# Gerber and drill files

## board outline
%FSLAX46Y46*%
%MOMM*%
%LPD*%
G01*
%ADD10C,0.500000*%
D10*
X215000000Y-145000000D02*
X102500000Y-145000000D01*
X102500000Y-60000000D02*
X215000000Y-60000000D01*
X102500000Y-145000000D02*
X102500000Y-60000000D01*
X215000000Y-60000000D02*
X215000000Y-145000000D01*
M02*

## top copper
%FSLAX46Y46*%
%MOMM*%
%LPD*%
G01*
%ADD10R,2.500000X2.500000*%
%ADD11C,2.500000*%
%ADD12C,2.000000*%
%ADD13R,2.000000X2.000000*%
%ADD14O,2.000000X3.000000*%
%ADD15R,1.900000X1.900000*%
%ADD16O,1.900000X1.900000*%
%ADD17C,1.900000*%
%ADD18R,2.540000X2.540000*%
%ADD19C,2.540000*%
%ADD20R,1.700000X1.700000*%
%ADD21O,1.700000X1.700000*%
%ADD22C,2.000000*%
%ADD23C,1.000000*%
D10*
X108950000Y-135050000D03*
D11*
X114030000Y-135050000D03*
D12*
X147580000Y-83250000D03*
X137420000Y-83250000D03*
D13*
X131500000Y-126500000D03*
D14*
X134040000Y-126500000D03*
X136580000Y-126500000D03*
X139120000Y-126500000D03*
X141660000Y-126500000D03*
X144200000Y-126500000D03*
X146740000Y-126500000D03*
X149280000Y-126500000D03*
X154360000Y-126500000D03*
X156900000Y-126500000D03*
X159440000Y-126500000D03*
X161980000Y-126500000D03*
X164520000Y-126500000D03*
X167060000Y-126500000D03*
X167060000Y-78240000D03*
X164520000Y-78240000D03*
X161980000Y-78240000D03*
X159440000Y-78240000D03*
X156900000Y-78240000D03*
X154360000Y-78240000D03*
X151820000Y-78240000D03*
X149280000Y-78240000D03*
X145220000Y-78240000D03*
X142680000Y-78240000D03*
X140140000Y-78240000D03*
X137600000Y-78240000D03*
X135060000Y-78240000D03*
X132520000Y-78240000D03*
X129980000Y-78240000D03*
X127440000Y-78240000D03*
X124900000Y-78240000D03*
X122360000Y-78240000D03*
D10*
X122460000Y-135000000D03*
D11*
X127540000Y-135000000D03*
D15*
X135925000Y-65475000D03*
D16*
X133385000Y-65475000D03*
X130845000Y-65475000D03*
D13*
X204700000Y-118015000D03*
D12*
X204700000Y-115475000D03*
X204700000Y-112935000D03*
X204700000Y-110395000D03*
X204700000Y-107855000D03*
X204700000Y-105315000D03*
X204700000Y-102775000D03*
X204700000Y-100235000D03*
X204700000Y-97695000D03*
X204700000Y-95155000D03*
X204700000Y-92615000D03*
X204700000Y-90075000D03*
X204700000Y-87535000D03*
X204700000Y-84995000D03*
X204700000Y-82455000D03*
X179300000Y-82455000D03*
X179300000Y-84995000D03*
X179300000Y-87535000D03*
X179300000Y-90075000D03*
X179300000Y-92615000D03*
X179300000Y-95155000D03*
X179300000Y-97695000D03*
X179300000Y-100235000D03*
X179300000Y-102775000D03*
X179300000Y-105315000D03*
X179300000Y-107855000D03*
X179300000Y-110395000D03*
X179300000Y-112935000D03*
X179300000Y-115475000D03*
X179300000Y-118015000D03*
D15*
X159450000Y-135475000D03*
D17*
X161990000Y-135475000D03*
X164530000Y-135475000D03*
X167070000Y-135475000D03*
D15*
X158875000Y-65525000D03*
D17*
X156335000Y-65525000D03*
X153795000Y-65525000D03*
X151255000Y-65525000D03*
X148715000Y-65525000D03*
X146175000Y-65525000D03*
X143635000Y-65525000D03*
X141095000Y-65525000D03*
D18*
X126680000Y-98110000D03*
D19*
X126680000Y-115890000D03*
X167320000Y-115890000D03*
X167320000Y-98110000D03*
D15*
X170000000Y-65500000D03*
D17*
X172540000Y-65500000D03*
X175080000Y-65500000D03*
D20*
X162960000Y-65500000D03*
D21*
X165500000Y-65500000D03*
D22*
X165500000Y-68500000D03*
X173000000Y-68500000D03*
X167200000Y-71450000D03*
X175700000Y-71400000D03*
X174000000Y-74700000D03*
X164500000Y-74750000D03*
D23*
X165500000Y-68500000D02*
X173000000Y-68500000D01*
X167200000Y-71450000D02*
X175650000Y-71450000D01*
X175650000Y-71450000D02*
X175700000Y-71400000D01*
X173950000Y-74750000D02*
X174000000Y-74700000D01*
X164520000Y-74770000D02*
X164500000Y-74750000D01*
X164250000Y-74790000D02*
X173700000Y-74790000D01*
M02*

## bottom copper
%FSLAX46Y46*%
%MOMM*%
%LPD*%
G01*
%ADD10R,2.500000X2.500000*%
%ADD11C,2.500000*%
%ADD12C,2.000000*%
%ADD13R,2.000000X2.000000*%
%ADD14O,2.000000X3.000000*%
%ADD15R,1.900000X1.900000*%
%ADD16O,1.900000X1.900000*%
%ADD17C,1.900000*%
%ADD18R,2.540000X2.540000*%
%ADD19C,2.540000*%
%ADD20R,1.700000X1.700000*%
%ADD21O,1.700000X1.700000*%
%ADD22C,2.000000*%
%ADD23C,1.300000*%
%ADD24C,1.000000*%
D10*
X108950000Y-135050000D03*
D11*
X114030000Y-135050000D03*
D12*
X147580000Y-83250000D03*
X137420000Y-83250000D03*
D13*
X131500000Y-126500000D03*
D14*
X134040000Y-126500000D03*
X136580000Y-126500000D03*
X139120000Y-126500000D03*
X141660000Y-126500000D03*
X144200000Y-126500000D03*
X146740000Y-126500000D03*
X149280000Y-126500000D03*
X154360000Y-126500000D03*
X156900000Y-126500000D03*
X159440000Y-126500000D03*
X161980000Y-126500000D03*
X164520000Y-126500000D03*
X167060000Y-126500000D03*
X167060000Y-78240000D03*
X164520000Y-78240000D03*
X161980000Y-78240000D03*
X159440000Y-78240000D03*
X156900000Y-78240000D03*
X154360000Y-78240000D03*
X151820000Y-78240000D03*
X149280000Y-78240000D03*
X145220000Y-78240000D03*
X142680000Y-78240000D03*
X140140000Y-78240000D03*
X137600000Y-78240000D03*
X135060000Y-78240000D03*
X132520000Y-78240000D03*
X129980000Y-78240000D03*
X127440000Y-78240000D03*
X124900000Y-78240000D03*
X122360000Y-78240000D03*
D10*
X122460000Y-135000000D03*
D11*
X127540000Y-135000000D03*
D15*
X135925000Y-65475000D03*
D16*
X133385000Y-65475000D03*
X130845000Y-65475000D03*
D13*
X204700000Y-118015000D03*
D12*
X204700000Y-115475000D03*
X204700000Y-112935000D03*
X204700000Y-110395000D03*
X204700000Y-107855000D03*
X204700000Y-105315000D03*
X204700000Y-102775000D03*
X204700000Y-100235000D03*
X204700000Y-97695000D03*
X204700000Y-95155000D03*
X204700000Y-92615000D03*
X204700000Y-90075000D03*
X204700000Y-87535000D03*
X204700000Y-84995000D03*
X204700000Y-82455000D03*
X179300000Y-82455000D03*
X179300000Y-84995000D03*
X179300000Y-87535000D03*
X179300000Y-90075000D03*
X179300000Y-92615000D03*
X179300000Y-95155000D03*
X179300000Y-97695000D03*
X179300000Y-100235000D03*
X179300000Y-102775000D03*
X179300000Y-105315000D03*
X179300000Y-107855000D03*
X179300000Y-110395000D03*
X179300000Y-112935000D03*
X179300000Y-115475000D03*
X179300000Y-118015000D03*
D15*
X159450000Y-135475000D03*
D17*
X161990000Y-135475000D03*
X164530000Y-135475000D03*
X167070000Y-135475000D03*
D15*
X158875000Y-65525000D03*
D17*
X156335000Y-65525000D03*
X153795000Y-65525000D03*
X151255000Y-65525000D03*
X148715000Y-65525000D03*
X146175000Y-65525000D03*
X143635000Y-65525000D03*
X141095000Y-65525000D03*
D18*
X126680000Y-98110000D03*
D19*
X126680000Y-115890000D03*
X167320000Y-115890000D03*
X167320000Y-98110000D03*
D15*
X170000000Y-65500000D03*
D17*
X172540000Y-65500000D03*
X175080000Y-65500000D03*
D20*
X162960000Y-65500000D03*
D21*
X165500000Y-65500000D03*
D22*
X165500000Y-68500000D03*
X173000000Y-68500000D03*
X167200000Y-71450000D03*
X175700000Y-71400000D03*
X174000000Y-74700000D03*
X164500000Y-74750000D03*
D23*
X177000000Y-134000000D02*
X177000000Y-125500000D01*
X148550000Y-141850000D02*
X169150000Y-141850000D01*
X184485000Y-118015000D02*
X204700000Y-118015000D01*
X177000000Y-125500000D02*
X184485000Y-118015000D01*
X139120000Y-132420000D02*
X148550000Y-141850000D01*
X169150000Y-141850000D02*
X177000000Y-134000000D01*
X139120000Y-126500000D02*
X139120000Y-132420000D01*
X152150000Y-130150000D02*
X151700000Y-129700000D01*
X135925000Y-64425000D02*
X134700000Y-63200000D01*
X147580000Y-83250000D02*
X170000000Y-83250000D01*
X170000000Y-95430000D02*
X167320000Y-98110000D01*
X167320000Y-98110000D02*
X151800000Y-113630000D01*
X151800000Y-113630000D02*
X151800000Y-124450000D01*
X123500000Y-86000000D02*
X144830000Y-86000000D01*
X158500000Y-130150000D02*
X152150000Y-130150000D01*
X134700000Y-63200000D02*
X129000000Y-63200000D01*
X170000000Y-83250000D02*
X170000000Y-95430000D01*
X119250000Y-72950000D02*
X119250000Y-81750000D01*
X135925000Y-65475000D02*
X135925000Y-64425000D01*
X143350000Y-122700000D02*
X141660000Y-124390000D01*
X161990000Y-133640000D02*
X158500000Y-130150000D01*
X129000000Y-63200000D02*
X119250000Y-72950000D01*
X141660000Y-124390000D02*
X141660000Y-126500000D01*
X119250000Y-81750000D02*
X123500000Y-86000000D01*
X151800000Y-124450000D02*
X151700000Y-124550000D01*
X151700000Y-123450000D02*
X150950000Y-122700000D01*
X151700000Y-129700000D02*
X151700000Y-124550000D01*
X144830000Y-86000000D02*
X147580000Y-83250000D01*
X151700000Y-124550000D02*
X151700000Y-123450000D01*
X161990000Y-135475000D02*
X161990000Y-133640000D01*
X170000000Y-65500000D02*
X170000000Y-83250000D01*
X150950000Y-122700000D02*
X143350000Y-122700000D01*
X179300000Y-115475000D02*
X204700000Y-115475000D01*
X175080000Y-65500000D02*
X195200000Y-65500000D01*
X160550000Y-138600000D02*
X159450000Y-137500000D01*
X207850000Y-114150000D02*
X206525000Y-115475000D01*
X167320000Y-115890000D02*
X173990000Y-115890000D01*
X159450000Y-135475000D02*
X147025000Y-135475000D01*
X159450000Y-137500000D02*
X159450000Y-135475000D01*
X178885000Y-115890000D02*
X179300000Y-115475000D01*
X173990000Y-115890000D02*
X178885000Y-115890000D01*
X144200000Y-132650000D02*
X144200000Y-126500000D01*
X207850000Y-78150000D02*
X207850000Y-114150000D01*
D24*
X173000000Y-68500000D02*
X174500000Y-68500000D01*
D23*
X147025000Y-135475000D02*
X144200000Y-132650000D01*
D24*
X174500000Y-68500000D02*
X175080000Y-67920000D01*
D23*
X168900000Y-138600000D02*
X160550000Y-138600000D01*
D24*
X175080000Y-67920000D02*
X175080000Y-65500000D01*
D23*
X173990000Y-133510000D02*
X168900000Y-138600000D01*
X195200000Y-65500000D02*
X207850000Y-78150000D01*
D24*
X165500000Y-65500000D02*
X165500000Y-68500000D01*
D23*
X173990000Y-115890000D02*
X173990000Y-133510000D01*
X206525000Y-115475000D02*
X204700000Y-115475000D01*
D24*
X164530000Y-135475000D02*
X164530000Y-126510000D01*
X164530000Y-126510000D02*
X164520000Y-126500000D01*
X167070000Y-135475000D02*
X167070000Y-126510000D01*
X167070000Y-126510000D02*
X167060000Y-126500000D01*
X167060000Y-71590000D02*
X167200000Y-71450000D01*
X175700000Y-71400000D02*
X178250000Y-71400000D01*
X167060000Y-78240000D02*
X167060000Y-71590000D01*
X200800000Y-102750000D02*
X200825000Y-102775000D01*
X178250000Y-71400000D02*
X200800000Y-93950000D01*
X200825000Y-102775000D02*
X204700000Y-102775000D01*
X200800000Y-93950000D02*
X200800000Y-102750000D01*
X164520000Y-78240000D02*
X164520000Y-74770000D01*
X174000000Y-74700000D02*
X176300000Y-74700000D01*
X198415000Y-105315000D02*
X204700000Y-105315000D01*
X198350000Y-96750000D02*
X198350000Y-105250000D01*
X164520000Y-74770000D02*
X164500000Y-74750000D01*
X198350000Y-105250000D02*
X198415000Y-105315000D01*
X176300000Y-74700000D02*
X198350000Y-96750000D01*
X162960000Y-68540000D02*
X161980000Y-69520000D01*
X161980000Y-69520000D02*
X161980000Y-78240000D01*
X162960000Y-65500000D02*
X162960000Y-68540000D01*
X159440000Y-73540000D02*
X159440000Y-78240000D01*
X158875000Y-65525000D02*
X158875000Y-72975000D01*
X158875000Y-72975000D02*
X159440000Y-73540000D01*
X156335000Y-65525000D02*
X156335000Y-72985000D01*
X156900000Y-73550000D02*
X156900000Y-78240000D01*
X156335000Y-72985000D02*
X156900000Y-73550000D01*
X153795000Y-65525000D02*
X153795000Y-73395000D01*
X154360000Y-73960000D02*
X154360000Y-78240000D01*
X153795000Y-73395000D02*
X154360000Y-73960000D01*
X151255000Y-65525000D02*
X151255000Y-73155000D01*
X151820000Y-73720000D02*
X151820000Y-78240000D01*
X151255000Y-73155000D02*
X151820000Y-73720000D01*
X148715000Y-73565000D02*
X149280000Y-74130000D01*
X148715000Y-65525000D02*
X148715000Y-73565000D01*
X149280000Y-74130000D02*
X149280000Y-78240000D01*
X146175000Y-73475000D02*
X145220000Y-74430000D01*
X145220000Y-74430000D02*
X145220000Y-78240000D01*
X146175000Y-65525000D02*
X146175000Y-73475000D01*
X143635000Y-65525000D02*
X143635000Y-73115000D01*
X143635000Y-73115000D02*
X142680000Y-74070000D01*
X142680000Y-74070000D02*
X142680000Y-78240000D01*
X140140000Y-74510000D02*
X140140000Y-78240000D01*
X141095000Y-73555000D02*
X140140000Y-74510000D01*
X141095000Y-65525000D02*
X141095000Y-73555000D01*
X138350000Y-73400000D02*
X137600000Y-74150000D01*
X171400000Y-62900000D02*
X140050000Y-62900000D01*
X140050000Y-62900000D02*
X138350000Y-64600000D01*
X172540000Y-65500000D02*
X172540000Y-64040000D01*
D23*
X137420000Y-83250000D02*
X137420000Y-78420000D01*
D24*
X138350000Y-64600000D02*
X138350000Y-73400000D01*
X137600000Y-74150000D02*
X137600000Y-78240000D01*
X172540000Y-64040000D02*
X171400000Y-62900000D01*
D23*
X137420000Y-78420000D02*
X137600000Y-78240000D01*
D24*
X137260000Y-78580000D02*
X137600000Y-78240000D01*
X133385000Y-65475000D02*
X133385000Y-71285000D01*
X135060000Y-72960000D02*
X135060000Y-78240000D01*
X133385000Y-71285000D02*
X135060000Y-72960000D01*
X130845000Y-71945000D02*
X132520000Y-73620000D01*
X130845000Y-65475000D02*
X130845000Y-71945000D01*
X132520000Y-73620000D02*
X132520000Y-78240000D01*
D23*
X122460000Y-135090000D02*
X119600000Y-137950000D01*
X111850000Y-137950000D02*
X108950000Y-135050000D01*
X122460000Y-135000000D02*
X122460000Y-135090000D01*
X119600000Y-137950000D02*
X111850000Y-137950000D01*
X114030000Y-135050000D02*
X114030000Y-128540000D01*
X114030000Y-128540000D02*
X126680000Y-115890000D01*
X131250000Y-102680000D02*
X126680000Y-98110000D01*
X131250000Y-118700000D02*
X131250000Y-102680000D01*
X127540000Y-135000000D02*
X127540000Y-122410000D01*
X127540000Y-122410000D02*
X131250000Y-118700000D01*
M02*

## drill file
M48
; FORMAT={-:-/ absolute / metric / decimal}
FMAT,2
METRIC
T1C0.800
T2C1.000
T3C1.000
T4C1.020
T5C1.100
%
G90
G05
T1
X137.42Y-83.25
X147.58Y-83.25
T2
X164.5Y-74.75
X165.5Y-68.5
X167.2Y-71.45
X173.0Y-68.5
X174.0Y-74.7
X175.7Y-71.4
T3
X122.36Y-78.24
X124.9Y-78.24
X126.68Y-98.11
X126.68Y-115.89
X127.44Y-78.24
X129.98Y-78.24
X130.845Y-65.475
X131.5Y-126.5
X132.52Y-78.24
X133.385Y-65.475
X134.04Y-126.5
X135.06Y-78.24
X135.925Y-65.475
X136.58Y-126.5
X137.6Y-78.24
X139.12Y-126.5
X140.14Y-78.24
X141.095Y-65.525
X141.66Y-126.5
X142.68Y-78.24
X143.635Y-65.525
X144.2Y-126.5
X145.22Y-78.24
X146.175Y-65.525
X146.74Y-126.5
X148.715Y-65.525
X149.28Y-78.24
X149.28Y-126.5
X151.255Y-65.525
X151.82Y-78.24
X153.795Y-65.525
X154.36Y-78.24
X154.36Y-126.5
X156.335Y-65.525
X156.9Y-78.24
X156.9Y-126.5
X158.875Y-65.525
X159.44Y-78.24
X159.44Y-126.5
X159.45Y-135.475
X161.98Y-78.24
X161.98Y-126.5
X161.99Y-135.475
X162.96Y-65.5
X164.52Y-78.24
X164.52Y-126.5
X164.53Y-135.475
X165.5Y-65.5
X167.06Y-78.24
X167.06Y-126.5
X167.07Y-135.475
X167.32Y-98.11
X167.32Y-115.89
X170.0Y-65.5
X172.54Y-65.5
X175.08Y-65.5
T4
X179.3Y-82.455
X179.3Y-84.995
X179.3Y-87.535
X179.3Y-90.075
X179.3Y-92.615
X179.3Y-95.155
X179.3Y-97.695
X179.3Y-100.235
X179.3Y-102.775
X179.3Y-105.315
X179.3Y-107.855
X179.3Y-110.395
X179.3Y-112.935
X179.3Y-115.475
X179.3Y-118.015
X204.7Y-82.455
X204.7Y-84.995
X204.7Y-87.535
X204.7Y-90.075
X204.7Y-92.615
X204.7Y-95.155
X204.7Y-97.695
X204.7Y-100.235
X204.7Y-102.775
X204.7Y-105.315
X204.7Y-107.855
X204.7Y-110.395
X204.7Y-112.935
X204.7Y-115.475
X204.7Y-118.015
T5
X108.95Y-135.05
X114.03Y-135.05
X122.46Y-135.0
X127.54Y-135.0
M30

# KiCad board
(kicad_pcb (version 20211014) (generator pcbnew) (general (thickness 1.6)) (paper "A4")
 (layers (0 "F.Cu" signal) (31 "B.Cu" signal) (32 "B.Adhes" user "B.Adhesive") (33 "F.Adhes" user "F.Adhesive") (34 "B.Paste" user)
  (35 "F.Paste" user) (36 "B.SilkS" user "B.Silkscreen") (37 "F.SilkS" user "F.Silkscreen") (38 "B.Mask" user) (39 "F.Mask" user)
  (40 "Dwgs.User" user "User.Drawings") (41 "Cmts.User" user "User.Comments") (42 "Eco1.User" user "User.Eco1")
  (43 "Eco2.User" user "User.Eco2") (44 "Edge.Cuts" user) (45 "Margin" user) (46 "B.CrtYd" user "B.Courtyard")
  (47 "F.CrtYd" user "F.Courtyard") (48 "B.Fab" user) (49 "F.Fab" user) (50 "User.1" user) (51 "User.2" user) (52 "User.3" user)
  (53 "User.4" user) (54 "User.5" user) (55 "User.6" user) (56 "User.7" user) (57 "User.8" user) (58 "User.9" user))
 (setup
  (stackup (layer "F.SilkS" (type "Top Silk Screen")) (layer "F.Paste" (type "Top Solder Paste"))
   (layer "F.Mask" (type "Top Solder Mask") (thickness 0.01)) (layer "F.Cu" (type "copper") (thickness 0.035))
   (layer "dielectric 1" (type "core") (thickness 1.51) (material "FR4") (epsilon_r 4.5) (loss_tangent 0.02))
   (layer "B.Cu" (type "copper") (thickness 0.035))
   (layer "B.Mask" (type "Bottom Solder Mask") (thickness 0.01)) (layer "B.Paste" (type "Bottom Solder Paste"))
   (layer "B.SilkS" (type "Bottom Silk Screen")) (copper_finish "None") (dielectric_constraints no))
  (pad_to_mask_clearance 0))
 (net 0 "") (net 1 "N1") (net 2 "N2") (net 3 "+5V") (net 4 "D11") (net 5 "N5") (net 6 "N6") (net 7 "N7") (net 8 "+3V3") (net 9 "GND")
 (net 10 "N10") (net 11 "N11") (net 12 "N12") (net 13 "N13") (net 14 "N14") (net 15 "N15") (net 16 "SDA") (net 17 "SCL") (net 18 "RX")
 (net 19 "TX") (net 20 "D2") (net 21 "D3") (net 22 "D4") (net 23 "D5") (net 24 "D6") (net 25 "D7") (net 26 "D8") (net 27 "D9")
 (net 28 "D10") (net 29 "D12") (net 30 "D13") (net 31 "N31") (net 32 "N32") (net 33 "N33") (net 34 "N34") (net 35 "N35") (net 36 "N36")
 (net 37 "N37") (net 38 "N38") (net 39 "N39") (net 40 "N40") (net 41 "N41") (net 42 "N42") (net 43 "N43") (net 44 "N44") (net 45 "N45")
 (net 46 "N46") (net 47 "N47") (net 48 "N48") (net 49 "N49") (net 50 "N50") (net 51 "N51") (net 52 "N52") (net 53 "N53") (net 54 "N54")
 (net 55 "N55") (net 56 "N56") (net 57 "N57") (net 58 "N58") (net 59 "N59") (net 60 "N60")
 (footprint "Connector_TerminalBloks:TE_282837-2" (layer "F.Cu") (at 111.49 135.05)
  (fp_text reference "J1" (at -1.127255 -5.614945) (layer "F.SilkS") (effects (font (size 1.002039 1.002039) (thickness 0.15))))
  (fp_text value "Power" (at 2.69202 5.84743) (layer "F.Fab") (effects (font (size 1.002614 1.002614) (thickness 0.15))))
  (pad "1" thru_hole rect (at -2.54 0) (size 2.5 2.5) (drill 1.1) (layers *.Cu *.Mask) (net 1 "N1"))
  (pad "2" thru_hole circle (at 2.54 0) (size 2.5 2.5) (drill 1.1) (layers *.Cu *.Mask) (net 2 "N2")))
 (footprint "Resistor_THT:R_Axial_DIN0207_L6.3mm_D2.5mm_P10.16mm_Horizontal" (layer "F.Cu") (at 147.58 83.25 180)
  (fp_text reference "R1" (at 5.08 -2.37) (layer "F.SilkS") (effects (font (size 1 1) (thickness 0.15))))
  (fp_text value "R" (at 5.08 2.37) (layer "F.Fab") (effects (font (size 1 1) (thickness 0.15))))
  (pad "1" thru_hole circle (at 0 0 180) (size 2 2) (drill 0.8) (layers *.Cu *.Mask) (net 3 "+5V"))
  (pad "2" thru_hole circle (at 10.16 0 180) (size 2 2) (drill 0.8) (layers *.Cu *.Mask) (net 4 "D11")))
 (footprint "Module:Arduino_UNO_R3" (layer "F.Cu") (at 131.5 80.5)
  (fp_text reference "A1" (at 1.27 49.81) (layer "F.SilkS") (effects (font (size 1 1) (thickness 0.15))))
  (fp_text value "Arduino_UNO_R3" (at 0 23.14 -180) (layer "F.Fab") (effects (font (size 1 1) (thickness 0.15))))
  (pad "1" thru_hole rect (at 0 46 90) (size 2 2) (drill 1) (layers *.Cu *.Mask) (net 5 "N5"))
  (pad "2" thru_hole oval (at 2.54 46 90) (size 3 2) (drill 1) (layers *.Cu *.Mask) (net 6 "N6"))
  (pad "3" thru_hole oval (at 5.08 46 90) (size 3 2) (drill 1) (layers *.Cu *.Mask) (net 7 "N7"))
  (pad "4" thru_hole oval (at 7.62 46 90) (size 3 2) (drill 1) (layers *.Cu *.Mask) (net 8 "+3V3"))
  (pad "5" thru_hole oval (at 10.16 46 90) (size 3 2) (drill 1) (layers *.Cu *.Mask) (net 3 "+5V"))
  (pad "6" thru_hole oval (at 12.7 46 90) (size 3 2) (drill 1) (layers *.Cu *.Mask) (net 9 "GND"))
  (pad "7" thru_hole oval (at 15.24 46 90) (size 3 2) (drill 1) (layers *.Cu *.Mask) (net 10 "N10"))
  (pad "8" thru_hole oval (at 17.78 46 90) (size 3 2) (drill 1) (layers *.Cu *.Mask) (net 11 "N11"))
  (pad "9" thru_hole oval (at 22.86 46 90) (size 3 2) (drill 1) (layers *.Cu *.Mask) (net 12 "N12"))
  (pad "10" thru_hole oval (at 25.4 46 90) (size 3 2) (drill 1) (layers *.Cu *.Mask) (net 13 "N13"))
  (pad "11" thru_hole oval (at 27.94 46 90) (size 3 2) (drill 1) (layers *.Cu *.Mask) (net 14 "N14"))
  (pad "12" thru_hole oval (at 30.48 46 90) (size 3 2) (drill 1) (layers *.Cu *.Mask) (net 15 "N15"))
  (pad "13" thru_hole oval (at 33.02 46 90) (size 3 2) (drill 1) (layers *.Cu *.Mask) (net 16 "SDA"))
  (pad "14" thru_hole oval (at 35.56 46 90) (size 3 2) (drill 1) (layers *.Cu *.Mask) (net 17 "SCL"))
  (pad "15" thru_hole oval (at 35.56 -2.26 90) (size 3 2) (drill 1) (layers *.Cu *.Mask) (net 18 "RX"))
  (pad "16" thru_hole oval (at 33.02 -2.26 90) (size 3 2) (drill 1) (layers *.Cu *.Mask) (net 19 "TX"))
  (pad "17" thru_hole oval (at 30.48 -2.26 90) (size 3 2) (drill 1) (layers *.Cu *.Mask) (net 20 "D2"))
  (pad "18" thru_hole oval (at 27.94 -2.26 90) (size 3 2) (drill 1) (layers *.Cu *.Mask) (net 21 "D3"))
  (pad "19" thru_hole oval (at 25.4 -2.26 90) (size 3 2) (drill 1) (layers *.Cu *.Mask) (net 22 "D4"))
  (pad "20" thru_hole oval (at 22.86 -2.26 90) (size 3 2) (drill 1) (layers *.Cu *.Mask) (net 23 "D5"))
  (pad "21" thru_hole oval (at 20.32 -2.26 90) (size 3 2) (drill 1) (layers *.Cu *.Mask) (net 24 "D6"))
  (pad "22" thru_hole oval (at 17.78 -2.26 90) (size 3 2) (drill 1) (layers *.Cu *.Mask) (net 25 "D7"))
  (pad "23" thru_hole oval (at 13.72 -2.26 90) (size 3 2) (drill 1) (layers *.Cu *.Mask) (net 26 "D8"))
  (pad "24" thru_hole oval (at 11.18 -2.26 90) (size 3 2) (drill 1) (layers *.Cu *.Mask) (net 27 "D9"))
  (pad "25" thru_hole oval (at 8.64 -2.26 90) (size 3 2) (drill 1) (layers *.Cu *.Mask) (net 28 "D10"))
  (pad "26" thru_hole oval (at 6.1 -2.26 90) (size 3 2) (drill 1) (layers *.Cu *.Mask) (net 4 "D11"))
  (pad "27" thru_hole oval (at 3.56 -2.26 90) (size 3 2) (drill 1) (layers *.Cu *.Mask) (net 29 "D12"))
  (pad "28" thru_hole oval (at 1.02 -2.26 90) (size 3 2) (drill 1) (layers *.Cu *.Mask) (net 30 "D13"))
  (pad "29" thru_hole oval (at -1.52 -2.26 90) (size 3 2) (drill 1) (layers *.Cu *.Mask) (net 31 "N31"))
  (pad "30" thru_hole oval (at -4.06 -2.26 90) (size 3 2) (drill 1) (layers *.Cu *.Mask) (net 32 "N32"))
  (pad "31" thru_hole oval (at -6.6 -2.26 90) (size 3 2) (drill 1) (layers *.Cu *.Mask) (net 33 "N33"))
  (pad "32" thru_hole oval (at -9.14 -2.26 90) (size 3 2) (drill 1) (layers *.Cu *.Mask) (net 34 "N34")))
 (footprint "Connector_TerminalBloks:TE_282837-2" (layer "F.Cu") (at 125 135)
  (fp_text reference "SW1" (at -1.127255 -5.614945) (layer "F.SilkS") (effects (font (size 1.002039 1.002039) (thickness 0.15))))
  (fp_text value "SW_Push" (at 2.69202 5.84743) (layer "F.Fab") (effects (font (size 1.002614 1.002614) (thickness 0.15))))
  (pad "1" thru_hole rect (at -2.54 0) (size 2.5 2.5) (drill 1.1) (layers *.Cu *.Mask) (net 1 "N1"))
  (pad "2" thru_hole circle (at 2.54 0) (size 2.5 2.5) (drill 1.1) (layers *.Cu *.Mask) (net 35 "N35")))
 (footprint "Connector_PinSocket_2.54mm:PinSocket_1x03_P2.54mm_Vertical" (layer "F.Cu") (at 135.925 65.475 -90)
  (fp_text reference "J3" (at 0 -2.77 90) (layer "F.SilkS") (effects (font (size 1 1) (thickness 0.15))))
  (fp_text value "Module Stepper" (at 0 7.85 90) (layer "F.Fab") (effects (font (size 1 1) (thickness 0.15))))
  (pad "1" thru_hole rect (at 0 0 270) (size 1.9 1.9) (drill 1) (layers *.Cu *.Mask) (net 3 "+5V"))
  (pad "2" thru_hole oval (at 0 2.54 270) (size 1.9 1.9) (drill 1) (layers *.Cu *.Mask) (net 29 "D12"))
  (pad "3" thru_hole oval (at 0 5.08 270) (size 1.9 1.9) (drill 1) (layers *.Cu *.Mask) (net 30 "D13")))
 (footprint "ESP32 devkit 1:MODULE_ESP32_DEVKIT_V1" (layer "F.Cu") (at 192 102.5 180)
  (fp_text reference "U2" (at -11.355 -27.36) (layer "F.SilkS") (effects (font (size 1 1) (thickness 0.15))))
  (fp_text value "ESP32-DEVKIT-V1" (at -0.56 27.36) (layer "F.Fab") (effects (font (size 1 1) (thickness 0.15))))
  (pad "1" thru_hole rect (at -12.7 -15.515 180) (size 2 2) (drill 1.02) (layers *.Cu *.Mask) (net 8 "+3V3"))
  (pad "2" thru_hole circle (at -12.7 -12.975 180) (size 2 2) (drill 1.02) (layers *.Cu *.Mask) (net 9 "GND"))
  (pad "3" thru_hole circle (at -12.7 -10.435 180) (size 2 2) (drill 1.02) (layers *.Cu *.Mask) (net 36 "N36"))
  (pad "4" thru_hole circle (at -12.7 -7.895 180) (size 2 2) (drill 1.02) (layers *.Cu *.Mask) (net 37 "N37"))
  (pad "5" thru_hole circle (at -12.7 -5.355 180) (size 2 2) (drill 1.02) (layers *.Cu *.Mask) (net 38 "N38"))
  (pad "6" thru_hole circle (at -12.7 -2.815 180) (size 2 2) (drill 1.02) (layers *.Cu *.Mask) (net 19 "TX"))
  (pad "7" thru_hole circle (at -12.7 -0.275 180) (size 2 2) (drill 1.02) (layers *.Cu *.Mask) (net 18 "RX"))
  (pad "8" thru_hole circle (at -12.7 2.265 180) (size 2 2) (drill 1.02) (layers *.Cu *.Mask) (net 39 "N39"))
  (pad "9" thru_hole circle (at -12.7 4.805 180) (size 2 2) (drill 1.02) (layers *.Cu *.Mask) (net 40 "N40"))
  (pad "10" thru_hole circle (at -12.7 7.345 180) (size 2 2) (drill 1.02) (layers *.Cu *.Mask) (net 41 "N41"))
  (pad "11" thru_hole circle (at -12.7 9.885 180) (size 2 2) (drill 1.02) (layers *.Cu *.Mask) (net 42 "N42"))
  (pad "12" thru_hole circle (at -12.7 12.425 180) (size 2 2) (drill 1.02) (layers *.Cu *.Mask) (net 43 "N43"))
  (pad "13" thru_hole circle (at -12.7 14.965 180) (size 2 2) (drill 1.02) (layers *.Cu *.Mask) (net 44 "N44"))
  (pad "14" thru_hole circle (at -12.7 17.505 180) (size 2 2) (drill 1.02) (layers *.Cu *.Mask) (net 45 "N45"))
  (pad "15" thru_hole circle (at -12.7 20.045 180) (size 2 2) (drill 1.02) (layers *.Cu *.Mask) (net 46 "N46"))
  (pad "16" thru_hole circle (at 12.7 20.045 180) (size 2 2) (drill 1.02) (layers *.Cu *.Mask) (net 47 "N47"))
  (pad "17" thru_hole circle (at 12.7 17.505 180) (size 2 2) (drill 1.02) (layers *.Cu *.Mask) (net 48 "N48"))
  (pad "18" thru_hole circle (at 12.7 14.965 180) (size 2 2) (drill 1.02) (layers *.Cu *.Mask) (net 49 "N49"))
  (pad "19" thru_hole circle (at 12.7 12.425 180) (size 2 2) (drill 1.02) (layers *.Cu *.Mask) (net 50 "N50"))
  (pad "20" thru_hole circle (at 12.7 9.885 180) (size 2 2) (drill 1.02) (layers *.Cu *.Mask) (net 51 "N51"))
  (pad "21" thru_hole circle (at 12.7 7.345 180) (size 2 2) (drill 1.02) (layers *.Cu *.Mask) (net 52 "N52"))
  (pad "22" thru_hole circle (at 12.7 4.805 180) (size 2 2) (drill 1.02) (layers *.Cu *.Mask) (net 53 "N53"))
  (pad "23" thru_hole circle (at 12.7 2.265 180) (size 2 2) (drill 1.02) (layers *.Cu *.Mask) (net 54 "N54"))
  (pad "24" thru_hole circle (at 12.7 -0.275 180) (size 2 2) (drill 1.02) (layers *.Cu *.Mask) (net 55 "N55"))
  (pad "25" thru_hole circle (at 12.7 -2.815 180) (size 2 2) (drill 1.02) (layers *.Cu *.Mask) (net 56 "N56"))
  (pad "26" thru_hole circle (at 12.7 -5.355 180) (size 2 2) (drill 1.02) (layers *.Cu *.Mask) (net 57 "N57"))
  (pad "27" thru_hole circle (at 12.7 -7.895 180) (size 2 2) (drill 1.02) (layers *.Cu *.Mask) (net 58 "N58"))
  (pad "28" thru_hole circle (at 12.7 -10.435 180) (size 2 2) (drill 1.02) (layers *.Cu *.Mask) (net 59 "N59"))
  (pad "29" thru_hole circle (at 12.7 -12.975 180) (size 2 2) (drill 1.02) (layers *.Cu *.Mask) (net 9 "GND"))
  (pad "30" thru_hole circle (at 12.7 -15.515 180) (size 2 2) (drill 1.02) (layers *.Cu *.Mask) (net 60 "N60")))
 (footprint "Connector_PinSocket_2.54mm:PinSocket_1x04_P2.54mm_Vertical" (layer "F.Cu") (at 159.45 135.475 90)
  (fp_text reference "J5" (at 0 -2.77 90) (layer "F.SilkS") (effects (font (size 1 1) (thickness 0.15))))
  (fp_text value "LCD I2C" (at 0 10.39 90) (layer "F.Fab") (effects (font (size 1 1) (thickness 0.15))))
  (pad "1" thru_hole rect (at 0 0 90) (size 1.9 1.9) (drill 1) (layers *.Cu *.Mask) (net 9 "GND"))
  (pad "2" thru_hole circle (at 0 2.54 90) (size 1.9 1.9) (drill 1) (layers *.Cu *.Mask) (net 3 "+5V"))
  (pad "3" thru_hole circle (at 0 5.08 90) (size 1.9 1.9) (drill 1) (layers *.Cu *.Mask) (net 16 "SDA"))
  (pad "4" thru_hole circle (at 0 7.62 90) (size 1.9 1.9) (drill 1) (layers *.Cu *.Mask) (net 17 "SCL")))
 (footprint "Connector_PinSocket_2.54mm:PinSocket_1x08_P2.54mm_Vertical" (layer "F.Cu") (at 158.875 65.525 -90)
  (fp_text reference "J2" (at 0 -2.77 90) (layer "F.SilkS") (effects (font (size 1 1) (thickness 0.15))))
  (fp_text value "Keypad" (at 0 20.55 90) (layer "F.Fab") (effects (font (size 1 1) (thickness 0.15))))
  (pad "1" thru_hole rect (at 0 0 270) (size 1.9 1.9) (drill 1) (layers *.Cu *.Mask) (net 21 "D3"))
  (pad "2" thru_hole circle (at 0 2.54 270) (size 1.9 1.9) (drill 1) (layers *.Cu *.Mask) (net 22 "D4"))
  (pad "3" thru_hole circle (at 0 5.08 270) (size 1.9 1.9) (drill 1) (layers *.Cu *.Mask) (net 23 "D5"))
  (pad "4" thru_hole circle (at 0 7.62 270) (size 1.9 1.9) (drill 1) (layers *.Cu *.Mask) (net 24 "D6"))
  (pad "5" thru_hole circle (at 0 10.16 270) (size 1.9 1.9) (drill 1) (layers *.Cu *.Mask) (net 25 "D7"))
  (pad "6" thru_hole circle (at 0 12.7 270) (size 1.9 1.9) (drill 1) (layers *.Cu *.Mask) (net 26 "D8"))
  (pad "7" thru_hole circle (at 0 15.24 270) (size 1.9 1.9) (drill 1) (layers *.Cu *.Mask) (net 27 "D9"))
  (pad "8" thru_hole circle (at 0 17.78 270) (size 1.9 1.9) (drill 1) (layers *.Cu *.Mask) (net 28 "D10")))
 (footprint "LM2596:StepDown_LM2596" (layer "F.Cu") (at 126.68 98.11)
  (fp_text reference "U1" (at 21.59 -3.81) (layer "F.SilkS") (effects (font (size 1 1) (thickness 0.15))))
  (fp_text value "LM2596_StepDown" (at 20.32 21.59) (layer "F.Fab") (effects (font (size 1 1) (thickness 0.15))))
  (pad "1" thru_hole rect (at 0 0) (size 2.54 2.54) (drill 1) (layers *.Cu *.Mask) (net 35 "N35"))
  (pad "2" thru_hole circle (at 0 17.78) (size 2.54 2.54) (drill 1) (layers *.Cu *.Mask) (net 2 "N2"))
  (pad "3" thru_hole circle (at 40.64 17.78) (size 2.54 2.54) (drill 1) (layers *.Cu *.Mask) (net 9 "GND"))
  (pad "4" thru_hole circle (at 40.64 0) (size 2.54 2.54) (drill 1) (layers *.Cu *.Mask) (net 3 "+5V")))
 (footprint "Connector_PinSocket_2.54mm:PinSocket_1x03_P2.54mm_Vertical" (layer "F.Cu") (at 170 65.5 90)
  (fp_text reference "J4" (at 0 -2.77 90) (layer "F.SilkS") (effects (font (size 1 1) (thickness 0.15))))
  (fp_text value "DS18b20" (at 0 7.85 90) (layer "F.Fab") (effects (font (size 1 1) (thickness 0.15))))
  (pad "1" thru_hole rect (at 0 0 90) (size 1.9 1.9) (drill 1) (layers *.Cu *.Mask) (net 3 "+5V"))
  (pad "2" thru_hole circle (at 0 2.54 90) (size 1.9 1.9) (drill 1) (layers *.Cu *.Mask) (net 4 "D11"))
  (pad "3" thru_hole circle (at 0 5.08 90) (size 1.9 1.9) (drill 1) (layers *.Cu *.Mask) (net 9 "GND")))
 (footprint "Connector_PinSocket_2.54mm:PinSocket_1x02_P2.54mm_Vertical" (layer "F.Cu") (at 162.96 65.5 90)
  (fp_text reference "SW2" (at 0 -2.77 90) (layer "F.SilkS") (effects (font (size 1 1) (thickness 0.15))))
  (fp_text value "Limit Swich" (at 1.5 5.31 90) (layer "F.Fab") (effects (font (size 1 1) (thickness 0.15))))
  (pad "1" thru_hole rect (at 0 0 90) (size 1.7 1.7) (drill 1) (layers *.Cu *.Mask) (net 20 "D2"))
  (pad "2" thru_hole oval (at 0 2.54 90) (size 1.7 1.7) (drill 1) (layers *.Cu *.Mask) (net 9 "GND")))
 (gr_line (start 215 145) (end 102.5 145) (layer "Edge.Cuts") (width 0.5))
 (gr_line (start 102.5 60) (end 215 60) (layer "Edge.Cuts") (width 0.5))
 (gr_line (start 102.5 145) (end 102.5 60) (layer "Edge.Cuts") (width 0.5))
 (gr_line (start 215 60) (end 215 145) (layer "Edge.Cuts") (width 0.5))
 (segment (start 177 134) (end 177 125.5) (width 1.3) (layer "B.Cu") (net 8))
 (segment (start 148.55 141.85) (end 169.15 141.85) (width 1.3) (layer "B.Cu") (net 8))
 (segment (start 184.485 118.015) (end 204.7 118.015) (width 1.3) (layer "B.Cu") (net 8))
 (segment (start 177 125.5) (end 184.485 118.015) (width 1.3) (layer "B.Cu") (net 8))
 (segment (start 139.12 132.42) (end 148.55 141.85) (width 1.3) (layer "B.Cu") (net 8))
 (segment (start 169.15 141.85) (end 177 134) (width 1.3) (layer "B.Cu") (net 8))
 (segment (start 139.12 126.5) (end 139.12 132.42) (width 1.3) (layer "B.Cu") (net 8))
 (segment (start 152.15 130.15) (end 151.7 129.7) (width 1.3) (layer "B.Cu") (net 3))
 (segment (start 135.925 64.425) (end 134.7 63.2) (width 1.3) (layer "B.Cu") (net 3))
 (segment (start 147.58 83.25) (end 170 83.25) (width 1.3) (layer "B.Cu") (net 3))
 (segment (start 170 95.43) (end 167.32 98.11) (width 1.3) (layer "B.Cu") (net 3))
 (segment (start 167.32 98.11) (end 151.8 113.63) (width 1.3) (layer "B.Cu") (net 3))
 (segment (start 151.8 113.63) (end 151.8 124.45) (width 1.3) (layer "B.Cu") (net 3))
 (segment (start 123.5 86) (end 144.83 86) (width 1.3) (layer "B.Cu") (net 3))
 (segment (start 158.5 130.15) (end 152.15 130.15) (width 1.3) (layer "B.Cu") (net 3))
 (segment (start 134.7 63.2) (end 129 63.2) (width 1.3) (layer "B.Cu") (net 3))
 (segment (start 170 83.25) (end 170 95.43) (width 1.3) (layer "B.Cu") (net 3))
 (segment (start 119.25 72.95) (end 119.25 81.75) (width 1.3) (layer "B.Cu") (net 3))
 (segment (start 135.925 65.475) (end 135.925 64.425) (width 1.3) (layer "B.Cu") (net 3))
 (segment (start 143.35 122.7) (end 141.66 124.39) (width 1.3) (layer "B.Cu") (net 3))
 (segment (start 161.99 133.64) (end 158.5 130.15) (width 1.3) (layer "B.Cu") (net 3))
 (segment (start 129 63.2) (end 119.25 72.95) (width 1.3) (layer "B.Cu") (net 3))
 (segment (start 141.66 124.39) (end 141.66 126.5) (width 1.3) (layer "B.Cu") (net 3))
 (segment (start 119.25 81.75) (end 123.5 86) (width 1.3) (layer "B.Cu") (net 3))
 (segment (start 151.8 124.45) (end 151.7 124.55) (width 1.3) (layer "B.Cu") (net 3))
 (segment (start 151.7 123.45) (end 150.95 122.7) (width 1.3) (layer "B.Cu") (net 3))
 (segment (start 151.7 129.7) (end 151.7 124.55) (width 1.3) (layer "B.Cu") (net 3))
 (segment (start 144.83 86) (end 147.58 83.25) (width 1.3) (layer "B.Cu") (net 3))
 (segment (start 151.7 124.55) (end 151.7 123.45) (width 1.3) (layer "B.Cu") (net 3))
 (segment (start 161.99 135.475) (end 161.99 133.64) (width 1.3) (layer "B.Cu") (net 3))
 (segment (start 170 65.5) (end 170 83.25) (width 1.3) (layer "B.Cu") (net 3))
 (segment (start 150.95 122.7) (end 143.35 122.7) (width 1.3) (layer "B.Cu") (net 3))
 (segment (start 165.5 68.5) (end 173 68.5) (width 1) (layer "F.Cu") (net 9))
 (via (at 165.5 68.5) (size 2) (drill 1) (layers "F.Cu" "B.Cu") (free) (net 9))
 (via (at 173 68.5) (size 2) (drill 1) (layers "F.Cu" "B.Cu") (free) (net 9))
 (segment (start 179.3 115.475) (end 204.7 115.475) (width 1.3) (layer "B.Cu") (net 9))
 (segment (start 175.08 65.5) (end 195.2 65.5) (width 1.3) (layer "B.Cu") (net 9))
 (segment (start 160.55 138.6) (end 159.45 137.5) (width 1.3) (layer "B.Cu") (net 9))
 (segment (start 207.85 114.15) (end 206.525 115.475) (width 1.3) (layer "B.Cu") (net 9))
 (segment (start 167.32 115.89) (end 173.99 115.89) (width 1.3) (layer "B.Cu") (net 9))
 (segment (start 159.45 135.475) (end 147.025 135.475) (width 1.3) (layer "B.Cu") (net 9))
 (segment (start 159.45 137.5) (end 159.45 135.475) (width 1.3) (layer "B.Cu") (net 9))
 (segment (start 178.885 115.89) (end 179.3 115.475) (width 1.3) (layer "B.Cu") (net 9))
 (segment (start 173.99 115.89) (end 178.885 115.89) (width 1.3) (layer "B.Cu") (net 9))
 (segment (start 144.2 132.65) (end 144.2 126.5) (width 1.3) (layer "B.Cu") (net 9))
 (segment (start 207.85 78.15) (end 207.85 114.15) (width 1.3) (layer "B.Cu") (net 9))
 (segment (start 173 68.5) (end 174.5 68.5) (width 1) (layer "B.Cu") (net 9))
 (segment (start 147.025 135.475) (end 144.2 132.65) (width 1.3) (layer "B.Cu") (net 9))
 (segment (start 174.5 68.5) (end 175.08 67.92) (width 1) (layer "B.Cu") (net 9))
 (segment (start 168.9 138.6) (end 160.55 138.6) (width 1.3) (layer "B.Cu") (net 9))
 (segment (start 175.08 67.92) (end 175.08 65.5) (width 1) (layer "B.Cu") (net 9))
 (segment (start 173.99 133.51) (end 168.9 138.6) (width 1.3) (layer "B.Cu") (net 9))
 (segment (start 195.2 65.5) (end 207.85 78.15) (width 1.3) (layer "B.Cu") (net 9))
 (segment (start 165.5 65.5) (end 165.5 68.5) (width 1) (layer "B.Cu") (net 9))
 (segment (start 173.99 115.89) (end 173.99 133.51) (width 1.3) (layer "B.Cu") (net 9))
 (segment (start 206.525 115.475) (end 204.7 115.475) (width 1.3) (layer "B.Cu") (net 9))
 (segment (start 164.53 135.475) (end 164.53 126.51) (width 1) (layer "B.Cu") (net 16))
 (segment (start 164.53 126.51) (end 164.52 126.5) (width 1) (layer "B.Cu") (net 16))
 (segment (start 167.07 135.475) (end 167.07 126.51) (width 1) (layer "B.Cu") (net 17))
 (segment (start 167.07 126.51) (end 167.06 126.5) (width 1) (layer "B.Cu") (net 17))
 (segment (start 167.2 71.45) (end 175.65 71.45) (width 1) (layer "F.Cu") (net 18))
 (segment (start 175.65 71.45) (end 175.7 71.4) (width 1) (layer "F.Cu") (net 18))
 (via (at 167.2 71.45) (size 2) (drill 1) (layers "F.Cu" "B.Cu") (free) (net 18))
 (via (at 175.7 71.4) (size 2) (drill 1) (layers "F.Cu" "B.Cu") (free) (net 18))
 (segment (start 167.06 71.59) (end 167.2 71.45) (width 1) (layer "B.Cu") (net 18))
 (segment (start 175.7 71.4) (end 178.25 71.4) (width 1) (layer "B.Cu") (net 18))
 (segment (start 167.06 78.24) (end 167.06 71.59) (width 1) (layer "B.Cu") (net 18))
 (segment (start 200.8 102.75) (end 200.825 102.775) (width 1) (layer "B.Cu") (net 18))
 (segment (start 178.25 71.4) (end 200.8 93.95) (width 1) (layer "B.Cu") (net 18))
 (segment (start 200.825 102.775) (end 204.7 102.775) (width 1) (layer "B.Cu") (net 18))
 (segment (start 200.8 93.95) (end 200.8 102.75) (width 1) (layer "B.Cu") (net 18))
 (segment (start 173.95 74.75) (end 174 74.7) (width 1) (layer "F.Cu") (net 19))
 (segment (start 164.52 74.77) (end 164.5 74.75) (width 1) (layer "F.Cu") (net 19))
 (segment (start 164.25 74.79) (end 173.7 74.79) (width 1) (layer "F.Cu") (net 19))
 (via (at 174 74.7) (size 2) (drill 1) (layers "F.Cu" "B.Cu") (free) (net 19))
 (via (at 164.5 74.75) (size 2) (drill 1) (layers "F.Cu" "B.Cu") (free) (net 19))
 (segment (start 164.52 78.24) (end 164.52 74.77) (width 1) (layer "B.Cu") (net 19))
 (segment (start 174 74.7) (end 176.3 74.7) (width 1) (layer "B.Cu") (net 19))
 (segment (start 198.415 105.315) (end 204.7 105.315) (width 1) (layer "B.Cu") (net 19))
 (segment (start 198.35 96.75) (end 198.35 105.25) (width 1) (layer "B.Cu") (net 19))
 (segment (start 164.52 74.77) (end 164.5 74.75) (width 1) (layer "B.Cu") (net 19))
 (segment (start 198.35 105.25) (end 198.415 105.315) (width 1) (layer "B.Cu") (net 19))
 (segment (start 176.3 74.7) (end 198.35 96.75) (width 1) (layer "B.Cu") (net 19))
 (segment (start 162.96 68.54) (end 161.98 69.52) (width 1) (layer "B.Cu") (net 20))
 (segment (start 161.98 69.52) (end 161.98 78.24) (width 1) (layer "B.Cu") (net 20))
 (segment (start 162.96 65.5) (end 162.96 68.54) (width 1) (layer "B.Cu") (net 20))
 (segment (start 159.44 73.54) (end 159.44 78.24) (width 1) (layer "B.Cu") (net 21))
 (segment (start 158.875 65.525) (end 158.875 72.975) (width 1) (layer "B.Cu") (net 21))
 (segment (start 158.875 72.975) (end 159.44 73.54) (width 1) (layer "B.Cu") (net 21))
 (segment (start 156.335 65.525) (end 156.335 72.985) (width 1) (layer "B.Cu") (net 22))
 (segment (start 156.9 73.55) (end 156.9 78.24) (width 1) (layer "B.Cu") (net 22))
 (segment (start 156.335 72.985) (end 156.9 73.55) (width 1) (layer "B.Cu") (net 22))
 (segment (start 153.795 65.525) (end 153.795 73.395) (width 1) (layer "B.Cu") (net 23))
 (segment (start 154.36 73.96) (end 154.36 78.24) (width 1) (layer "B.Cu") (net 23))
 (segment (start 153.795 73.395) (end 154.36 73.96) (width 1) (layer "B.Cu") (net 23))
 (segment (start 151.255 65.525) (end 151.255 73.155) (width 1) (layer "B.Cu") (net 24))
 (segment (start 151.82 73.72) (end 151.82 78.24) (width 1) (layer "B.Cu") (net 24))
 (segment (start 151.255 73.155) (end 151.82 73.72) (width 1) (layer "B.Cu") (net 24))
 (segment (start 148.715 73.565) (end 149.28 74.13) (width 1) (layer "B.Cu") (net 25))
 (segment (start 148.715 65.525) (end 148.715 73.565) (width 1) (layer "B.Cu") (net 25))
 (segment (start 149.28 74.13) (end 149.28 78.24) (width 1) (layer "B.Cu") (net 25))
 (segment (start 146.175 73.475) (end 145.22 74.43) (width 1) (layer "B.Cu") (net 26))
 (segment (start 145.22 74.43) (end 145.22 78.24) (width 1) (layer "B.Cu") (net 26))
 (segment (start 146.175 65.525) (end 146.175 73.475) (width 1) (layer "B.Cu") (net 26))
 (segment (start 143.635 65.525) (end 143.635 73.115) (width 1) (layer "B.Cu") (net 27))
 (segment (start 143.635 73.115) (end 142.68 74.07) (width 1) (layer "B.Cu") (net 27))
 (segment (start 142.68 74.07) (end 142.68 78.24) (width 1) (layer "B.Cu") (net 27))
 (segment (start 140.14 74.51) (end 140.14 78.24) (width 1) (layer "B.Cu") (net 28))
 (segment (start 141.095 73.555) (end 140.14 74.51) (width 1) (layer "B.Cu") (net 28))
 (segment (start 141.095 65.525) (end 141.095 73.555) (width 1) (layer "B.Cu") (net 28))
 (segment (start 138.35 73.4) (end 137.6 74.15) (width 1) (layer "B.Cu") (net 4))
 (segment (start 171.4 62.9) (end 140.05 62.9) (width 1) (layer "B.Cu") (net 4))
 (segment (start 140.05 62.9) (end 138.35 64.6) (width 1) (layer "B.Cu") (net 4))
 (segment (start 172.54 65.5) (end 172.54 64.04) (width 1) (layer "B.Cu") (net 4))
 (segment (start 137.42 83.25) (end 137.42 78.42) (width 1.3) (layer "B.Cu") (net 4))
 (segment (start 138.35 64.6) (end 138.35 73.4) (width 1) (layer "B.Cu") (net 4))
 (segment (start 137.6 74.15) (end 137.6 78.24) (width 1) (layer "B.Cu") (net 4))
 (segment (start 172.54 64.04) (end 171.4 62.9) (width 1) (layer "B.Cu") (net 4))
 (segment (start 137.42 78.42) (end 137.6 78.24) (width 1.3) (layer "B.Cu") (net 4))
 (segment (start 137.26 78.58) (end 137.6 78.24) (width 1) (layer "B.Cu") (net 4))
 (segment (start 133.385 65.475) (end 133.385 71.285) (width 1) (layer "B.Cu") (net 29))
 (segment (start 135.06 72.96) (end 135.06 78.24) (width 1) (layer "B.Cu") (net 29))
 (segment (start 133.385 71.285) (end 135.06 72.96) (width 1) (layer "B.Cu") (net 29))
 (segment (start 130.845 71.945) (end 132.52 73.62) (width 1) (layer "B.Cu") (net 30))
 (segment (start 130.845 65.475) (end 130.845 71.945) (width 1) (layer "B.Cu") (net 30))
 (segment (start 132.52 73.62) (end 132.52 78.24) (width 1) (layer "B.Cu") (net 30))
 (segment (start 122.46 135.09) (end 119.6 137.95) (width 1.3) (layer "B.Cu") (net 1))
 (segment (start 111.85 137.95) (end 108.95 135.05) (width 1.3) (layer "B.Cu") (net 1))
 (segment (start 122.46 135) (end 122.46 135.09) (width 1.3) (layer "B.Cu") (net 1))
 (segment (start 119.6 137.95) (end 111.85 137.95) (width 1.3) (layer "B.Cu") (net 1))
 (segment (start 114.03 135.05) (end 114.03 128.54) (width 1.3) (layer "B.Cu") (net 2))
 (segment (start 114.03 128.54) (end 126.68 115.89) (width 1.3) (layer "B.Cu") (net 2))
 (segment (start 131.25 102.68) (end 126.68 98.11) (width 1.3) (layer "B.Cu") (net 35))
 (segment (start 131.25 118.7) (end 131.25 102.68) (width 1.3) (layer "B.Cu") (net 35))
 (segment (start 127.54 135) (end 127.54 122.41) (width 1.3) (layer "B.Cu") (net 35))
 (segment (start 127.54 122.41) (end 131.25 118.7) (width 1.3) (layer "B.Cu") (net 35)))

